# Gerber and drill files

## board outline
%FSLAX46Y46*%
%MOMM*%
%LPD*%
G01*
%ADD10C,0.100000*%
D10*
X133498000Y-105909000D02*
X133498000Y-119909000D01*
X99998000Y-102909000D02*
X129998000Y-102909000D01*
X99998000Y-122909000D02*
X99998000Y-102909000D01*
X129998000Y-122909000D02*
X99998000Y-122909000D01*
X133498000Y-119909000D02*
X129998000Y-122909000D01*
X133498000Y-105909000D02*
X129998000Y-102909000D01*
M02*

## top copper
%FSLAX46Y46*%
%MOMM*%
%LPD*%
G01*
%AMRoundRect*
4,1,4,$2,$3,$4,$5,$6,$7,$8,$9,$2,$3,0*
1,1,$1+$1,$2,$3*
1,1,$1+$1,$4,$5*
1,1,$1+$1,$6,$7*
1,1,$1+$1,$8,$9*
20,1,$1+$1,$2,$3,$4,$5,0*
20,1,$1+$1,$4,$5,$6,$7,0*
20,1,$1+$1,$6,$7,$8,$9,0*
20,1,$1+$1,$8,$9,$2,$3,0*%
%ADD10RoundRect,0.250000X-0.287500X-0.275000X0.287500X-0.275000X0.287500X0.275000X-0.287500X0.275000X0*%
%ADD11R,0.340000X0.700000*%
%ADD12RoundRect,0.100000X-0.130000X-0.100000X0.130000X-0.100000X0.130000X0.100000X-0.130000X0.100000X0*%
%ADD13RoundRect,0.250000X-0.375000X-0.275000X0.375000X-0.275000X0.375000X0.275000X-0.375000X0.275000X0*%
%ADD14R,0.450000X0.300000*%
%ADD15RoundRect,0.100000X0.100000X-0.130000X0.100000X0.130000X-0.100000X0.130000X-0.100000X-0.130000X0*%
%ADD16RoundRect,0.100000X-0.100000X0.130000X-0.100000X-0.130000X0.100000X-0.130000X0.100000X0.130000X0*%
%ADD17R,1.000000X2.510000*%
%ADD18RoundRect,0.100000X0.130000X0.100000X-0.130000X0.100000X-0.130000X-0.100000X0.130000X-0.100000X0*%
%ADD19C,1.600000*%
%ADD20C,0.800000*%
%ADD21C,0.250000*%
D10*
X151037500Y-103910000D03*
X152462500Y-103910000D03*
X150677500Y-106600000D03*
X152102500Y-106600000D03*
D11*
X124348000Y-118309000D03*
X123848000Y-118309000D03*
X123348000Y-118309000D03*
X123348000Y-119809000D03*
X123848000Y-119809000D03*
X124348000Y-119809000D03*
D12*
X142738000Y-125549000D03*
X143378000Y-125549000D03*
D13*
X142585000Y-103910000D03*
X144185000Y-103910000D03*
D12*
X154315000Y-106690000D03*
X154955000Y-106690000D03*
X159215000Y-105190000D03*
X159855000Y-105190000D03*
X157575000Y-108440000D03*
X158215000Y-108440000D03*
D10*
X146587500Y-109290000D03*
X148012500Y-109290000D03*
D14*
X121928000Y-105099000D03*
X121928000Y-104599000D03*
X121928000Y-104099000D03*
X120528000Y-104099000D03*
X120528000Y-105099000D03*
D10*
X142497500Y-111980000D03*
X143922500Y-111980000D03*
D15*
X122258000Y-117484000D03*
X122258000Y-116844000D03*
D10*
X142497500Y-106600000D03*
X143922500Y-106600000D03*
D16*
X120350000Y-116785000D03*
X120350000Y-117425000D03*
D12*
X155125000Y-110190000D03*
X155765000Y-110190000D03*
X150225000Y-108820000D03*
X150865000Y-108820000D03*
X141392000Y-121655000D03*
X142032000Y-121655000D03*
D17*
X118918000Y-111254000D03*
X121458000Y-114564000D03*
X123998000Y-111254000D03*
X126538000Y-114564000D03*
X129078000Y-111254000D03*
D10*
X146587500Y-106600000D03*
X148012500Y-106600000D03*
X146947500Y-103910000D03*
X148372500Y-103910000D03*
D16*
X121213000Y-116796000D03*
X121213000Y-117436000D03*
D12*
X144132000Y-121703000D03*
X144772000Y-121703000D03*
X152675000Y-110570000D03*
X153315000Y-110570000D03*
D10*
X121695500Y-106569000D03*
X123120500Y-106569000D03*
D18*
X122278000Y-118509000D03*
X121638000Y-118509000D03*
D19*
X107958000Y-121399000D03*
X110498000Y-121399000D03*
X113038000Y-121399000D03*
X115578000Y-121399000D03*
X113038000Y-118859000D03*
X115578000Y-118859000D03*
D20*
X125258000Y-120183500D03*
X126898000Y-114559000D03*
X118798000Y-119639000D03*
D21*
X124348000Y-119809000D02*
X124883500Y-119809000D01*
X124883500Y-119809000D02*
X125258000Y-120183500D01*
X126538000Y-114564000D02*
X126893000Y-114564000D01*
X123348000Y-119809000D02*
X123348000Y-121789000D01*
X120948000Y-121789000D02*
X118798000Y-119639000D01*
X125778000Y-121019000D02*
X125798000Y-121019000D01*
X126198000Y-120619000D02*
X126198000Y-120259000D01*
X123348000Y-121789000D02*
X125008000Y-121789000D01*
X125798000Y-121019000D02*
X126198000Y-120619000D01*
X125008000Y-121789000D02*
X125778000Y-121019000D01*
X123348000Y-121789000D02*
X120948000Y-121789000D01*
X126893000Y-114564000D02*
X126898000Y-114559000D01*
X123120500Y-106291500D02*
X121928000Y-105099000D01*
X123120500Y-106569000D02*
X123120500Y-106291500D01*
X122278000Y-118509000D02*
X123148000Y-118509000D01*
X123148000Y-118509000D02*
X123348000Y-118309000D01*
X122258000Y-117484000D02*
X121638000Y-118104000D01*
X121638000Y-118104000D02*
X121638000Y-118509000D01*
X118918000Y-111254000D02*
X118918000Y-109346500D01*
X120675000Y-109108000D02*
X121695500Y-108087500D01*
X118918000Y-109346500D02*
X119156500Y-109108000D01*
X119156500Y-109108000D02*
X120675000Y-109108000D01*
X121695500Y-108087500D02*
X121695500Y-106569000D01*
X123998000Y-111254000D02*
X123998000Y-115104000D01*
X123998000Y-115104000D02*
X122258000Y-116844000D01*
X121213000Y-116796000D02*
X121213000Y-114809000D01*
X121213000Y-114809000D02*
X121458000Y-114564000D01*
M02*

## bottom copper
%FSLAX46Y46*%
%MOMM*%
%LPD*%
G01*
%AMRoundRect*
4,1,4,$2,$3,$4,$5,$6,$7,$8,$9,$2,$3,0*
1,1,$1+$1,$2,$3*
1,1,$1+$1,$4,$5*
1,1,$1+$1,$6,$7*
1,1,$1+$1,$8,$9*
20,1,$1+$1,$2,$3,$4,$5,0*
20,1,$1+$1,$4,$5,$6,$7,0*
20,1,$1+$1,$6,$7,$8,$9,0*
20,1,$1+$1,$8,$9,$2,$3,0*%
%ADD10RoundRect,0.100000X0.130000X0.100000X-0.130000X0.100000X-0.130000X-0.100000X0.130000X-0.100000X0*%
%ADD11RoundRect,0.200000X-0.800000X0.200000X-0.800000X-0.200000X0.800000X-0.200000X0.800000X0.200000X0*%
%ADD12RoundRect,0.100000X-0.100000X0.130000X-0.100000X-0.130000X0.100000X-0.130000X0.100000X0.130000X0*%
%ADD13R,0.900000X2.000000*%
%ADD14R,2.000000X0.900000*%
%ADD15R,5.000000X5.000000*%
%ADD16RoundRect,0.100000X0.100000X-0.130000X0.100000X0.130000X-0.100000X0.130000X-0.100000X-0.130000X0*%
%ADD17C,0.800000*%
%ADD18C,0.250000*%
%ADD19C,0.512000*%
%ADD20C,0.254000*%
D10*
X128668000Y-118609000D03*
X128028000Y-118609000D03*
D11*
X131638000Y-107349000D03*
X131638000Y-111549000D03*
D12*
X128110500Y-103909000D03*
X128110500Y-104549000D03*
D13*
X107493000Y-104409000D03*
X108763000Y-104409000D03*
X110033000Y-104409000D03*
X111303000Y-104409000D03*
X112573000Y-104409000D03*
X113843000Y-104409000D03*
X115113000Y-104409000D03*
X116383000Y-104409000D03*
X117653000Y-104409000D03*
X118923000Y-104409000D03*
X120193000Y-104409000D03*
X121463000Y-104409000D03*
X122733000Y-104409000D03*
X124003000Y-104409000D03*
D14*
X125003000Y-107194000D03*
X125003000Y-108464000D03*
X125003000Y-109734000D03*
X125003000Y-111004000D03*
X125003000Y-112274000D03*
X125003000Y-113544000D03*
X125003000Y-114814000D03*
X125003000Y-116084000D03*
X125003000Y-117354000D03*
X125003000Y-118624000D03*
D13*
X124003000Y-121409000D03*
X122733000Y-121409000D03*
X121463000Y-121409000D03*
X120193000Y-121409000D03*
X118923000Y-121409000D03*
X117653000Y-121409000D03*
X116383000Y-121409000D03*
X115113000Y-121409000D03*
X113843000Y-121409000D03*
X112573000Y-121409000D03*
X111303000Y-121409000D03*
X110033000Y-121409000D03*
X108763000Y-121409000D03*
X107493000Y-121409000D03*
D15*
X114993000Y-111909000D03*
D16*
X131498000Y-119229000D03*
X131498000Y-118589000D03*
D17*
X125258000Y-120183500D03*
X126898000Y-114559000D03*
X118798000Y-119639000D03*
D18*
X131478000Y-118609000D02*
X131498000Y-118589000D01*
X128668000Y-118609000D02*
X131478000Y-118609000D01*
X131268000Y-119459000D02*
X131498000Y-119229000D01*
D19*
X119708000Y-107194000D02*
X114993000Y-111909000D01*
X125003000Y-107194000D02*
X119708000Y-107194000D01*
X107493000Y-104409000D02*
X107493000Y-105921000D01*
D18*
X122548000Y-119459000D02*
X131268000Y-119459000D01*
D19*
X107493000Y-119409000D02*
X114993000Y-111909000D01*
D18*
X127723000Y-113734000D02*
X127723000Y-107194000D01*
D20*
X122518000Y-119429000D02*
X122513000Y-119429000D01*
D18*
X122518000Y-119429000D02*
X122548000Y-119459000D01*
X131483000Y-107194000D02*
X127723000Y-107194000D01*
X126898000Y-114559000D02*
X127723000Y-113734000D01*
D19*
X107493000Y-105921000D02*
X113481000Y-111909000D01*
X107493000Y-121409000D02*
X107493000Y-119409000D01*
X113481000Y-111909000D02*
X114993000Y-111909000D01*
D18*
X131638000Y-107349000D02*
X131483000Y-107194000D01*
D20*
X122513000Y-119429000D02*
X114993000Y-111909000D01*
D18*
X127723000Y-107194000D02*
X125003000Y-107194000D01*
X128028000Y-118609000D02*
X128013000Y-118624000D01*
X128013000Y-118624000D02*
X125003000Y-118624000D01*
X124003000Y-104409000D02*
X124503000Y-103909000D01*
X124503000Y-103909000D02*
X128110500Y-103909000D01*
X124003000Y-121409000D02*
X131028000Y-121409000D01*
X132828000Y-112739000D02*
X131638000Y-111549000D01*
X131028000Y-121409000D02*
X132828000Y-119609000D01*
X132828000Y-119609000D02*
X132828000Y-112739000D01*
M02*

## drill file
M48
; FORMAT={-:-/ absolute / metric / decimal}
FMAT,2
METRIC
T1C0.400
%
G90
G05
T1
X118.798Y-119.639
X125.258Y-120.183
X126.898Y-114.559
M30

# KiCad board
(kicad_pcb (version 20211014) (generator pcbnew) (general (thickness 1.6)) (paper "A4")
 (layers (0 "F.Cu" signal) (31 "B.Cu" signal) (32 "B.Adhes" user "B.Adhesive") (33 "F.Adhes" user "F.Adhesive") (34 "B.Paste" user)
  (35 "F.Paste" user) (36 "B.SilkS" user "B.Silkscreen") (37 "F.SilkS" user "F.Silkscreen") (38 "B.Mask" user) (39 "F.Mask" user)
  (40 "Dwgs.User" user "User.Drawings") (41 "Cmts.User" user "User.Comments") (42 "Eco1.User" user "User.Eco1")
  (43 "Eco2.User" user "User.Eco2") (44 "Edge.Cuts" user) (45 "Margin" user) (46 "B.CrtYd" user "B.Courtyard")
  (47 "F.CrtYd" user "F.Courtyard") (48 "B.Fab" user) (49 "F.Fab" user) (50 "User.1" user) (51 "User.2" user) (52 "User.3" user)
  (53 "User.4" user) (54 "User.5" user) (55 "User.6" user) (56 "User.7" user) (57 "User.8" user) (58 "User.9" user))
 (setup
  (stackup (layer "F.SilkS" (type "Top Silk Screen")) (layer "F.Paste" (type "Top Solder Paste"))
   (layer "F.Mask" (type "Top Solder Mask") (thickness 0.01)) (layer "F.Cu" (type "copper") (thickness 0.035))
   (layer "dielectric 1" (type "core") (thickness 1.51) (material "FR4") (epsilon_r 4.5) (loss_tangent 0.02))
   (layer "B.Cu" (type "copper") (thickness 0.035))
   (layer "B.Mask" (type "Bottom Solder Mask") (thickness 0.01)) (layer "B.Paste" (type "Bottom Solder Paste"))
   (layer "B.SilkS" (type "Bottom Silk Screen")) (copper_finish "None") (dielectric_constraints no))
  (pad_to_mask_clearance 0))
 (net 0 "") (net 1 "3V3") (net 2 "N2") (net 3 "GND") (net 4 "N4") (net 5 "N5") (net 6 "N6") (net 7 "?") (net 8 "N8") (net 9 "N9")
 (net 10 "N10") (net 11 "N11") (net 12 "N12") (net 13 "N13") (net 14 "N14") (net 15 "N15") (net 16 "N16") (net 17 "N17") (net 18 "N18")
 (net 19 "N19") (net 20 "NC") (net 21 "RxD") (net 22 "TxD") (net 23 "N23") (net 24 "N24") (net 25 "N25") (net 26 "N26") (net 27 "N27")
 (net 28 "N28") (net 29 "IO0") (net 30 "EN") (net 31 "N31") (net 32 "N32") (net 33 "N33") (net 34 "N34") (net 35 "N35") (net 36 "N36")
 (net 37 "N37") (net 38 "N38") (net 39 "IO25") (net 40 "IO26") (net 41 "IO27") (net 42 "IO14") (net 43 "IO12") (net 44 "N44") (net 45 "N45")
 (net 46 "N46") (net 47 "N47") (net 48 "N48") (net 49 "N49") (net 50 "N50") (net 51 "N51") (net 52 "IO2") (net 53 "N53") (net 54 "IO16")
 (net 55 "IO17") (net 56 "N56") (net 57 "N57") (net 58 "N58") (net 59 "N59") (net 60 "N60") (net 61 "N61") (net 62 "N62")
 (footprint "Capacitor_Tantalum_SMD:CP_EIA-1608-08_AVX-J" (layer "F.Cu") (at 151.75 103.91)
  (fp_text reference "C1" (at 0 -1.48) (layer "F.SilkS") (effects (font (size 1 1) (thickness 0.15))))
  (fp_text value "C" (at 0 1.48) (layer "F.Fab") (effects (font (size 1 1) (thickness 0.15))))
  (pad "1" smd roundrect (at -0.7125 0) (size 1.075 1.05) (layers "F.Cu" "F.Paste" "F.Mask") (roundrect_rratio 0.238095) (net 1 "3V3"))
  (pad "2" smd roundrect (at 0.7125 0) (size 1.075 1.05) (layers "F.Cu" "F.Paste" "F.Mask") (roundrect_rratio 0.238095) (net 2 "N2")))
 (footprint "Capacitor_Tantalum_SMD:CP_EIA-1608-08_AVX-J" (layer "F.Cu") (at 151.39 106.6)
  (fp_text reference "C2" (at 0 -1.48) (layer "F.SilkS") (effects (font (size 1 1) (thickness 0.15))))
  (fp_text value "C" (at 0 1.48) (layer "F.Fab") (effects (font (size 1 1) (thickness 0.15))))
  (pad "1" smd roundrect (at -0.7125 0) (size 1.075 1.05) (layers "F.Cu" "F.Paste" "F.Mask") (roundrect_rratio 0.238095) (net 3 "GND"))
  (pad "2" smd roundrect (at 0.7125 0) (size 1.075 1.05) (layers "F.Cu" "F.Paste" "F.Mask") (roundrect_rratio 0.238095) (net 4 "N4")))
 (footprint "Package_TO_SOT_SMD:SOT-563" (layer "F.Cu") (at 123.848 119.059 -90)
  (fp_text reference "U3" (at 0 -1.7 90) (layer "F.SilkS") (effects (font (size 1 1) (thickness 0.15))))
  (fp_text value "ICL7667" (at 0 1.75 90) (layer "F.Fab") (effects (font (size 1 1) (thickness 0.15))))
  (pad "1" smd rect (at -0.75 -0.5 270) (size 0.7 0.34) (layers "F.Cu" "F.Paste" "F.Mask") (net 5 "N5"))
  (pad "2" smd rect (at -0.75 0 270) (size 0.7 0.34) (layers "F.Cu" "F.Paste" "F.Mask") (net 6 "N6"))
  (pad "3" smd rect (at -0.75 0.5 270) (size 0.7 0.34) (layers "F.Cu" "F.Paste" "F.Mask") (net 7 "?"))
  (pad "4" smd rect (at 0.75 0.5 270) (size 0.7 0.34) (layers "F.Cu" "F.Paste" "F.Mask") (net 3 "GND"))
  (pad "5" smd rect (at 0.75 0 270) (size 0.7 0.34) (layers "F.Cu" "F.Paste" "F.Mask") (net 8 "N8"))
  (pad "6" smd rect (at 0.75 -0.5 270) (size 0.7 0.34) (layers "F.Cu" "F.Paste" "F.Mask") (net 1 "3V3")))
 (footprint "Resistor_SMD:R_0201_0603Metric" (layer "F.Cu") (at 143.058 125.549)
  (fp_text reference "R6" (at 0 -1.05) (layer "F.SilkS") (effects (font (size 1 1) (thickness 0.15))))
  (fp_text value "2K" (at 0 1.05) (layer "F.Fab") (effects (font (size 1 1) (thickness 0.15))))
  (pad "" smd roundrect (at -0.345 0) (size 0.318 0.36) (layers "F.Paste") (roundrect_rratio 0.25))
  (pad "" smd roundrect (at 0.345 0) (size 0.318 0.36) (layers "F.Paste") (roundrect_rratio 0.25))
  (pad "1" smd roundrect (at -0.32 0) (size 0.46 0.4) (layers "F.Cu" "F.Mask") (roundrect_rratio 0.25) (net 3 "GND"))
  (pad "2" smd roundrect (at 0.32 0) (size 0.46 0.4) (layers "F.Cu" "F.Mask") (roundrect_rratio 0.25) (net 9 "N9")))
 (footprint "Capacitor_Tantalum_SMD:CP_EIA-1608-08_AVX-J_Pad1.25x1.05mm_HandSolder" (layer "F.Cu") (at 143.385 103.91)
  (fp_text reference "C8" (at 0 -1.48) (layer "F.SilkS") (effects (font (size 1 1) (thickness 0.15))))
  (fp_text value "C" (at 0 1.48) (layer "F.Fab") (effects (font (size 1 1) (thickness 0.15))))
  (pad "1" smd roundrect (at -0.8 0) (size 1.25 1.05) (layers "F.Cu" "F.Paste" "F.Mask") (roundrect_rratio 0.238095) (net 1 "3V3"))
  (pad "2" smd roundrect (at 0.8 0) (size 1.25 1.05) (layers "F.Cu" "F.Paste" "F.Mask") (roundrect_rratio 0.238095) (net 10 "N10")))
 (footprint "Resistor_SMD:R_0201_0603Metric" (layer "F.Cu") (at 154.635 106.69)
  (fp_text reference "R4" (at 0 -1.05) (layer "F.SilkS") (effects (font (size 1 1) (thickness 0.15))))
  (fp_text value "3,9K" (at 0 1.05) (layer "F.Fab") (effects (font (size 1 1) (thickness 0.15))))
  (pad "" smd roundrect (at 0.345 0) (size 0.318 0.36) (layers "F.Paste") (roundrect_rratio 0.25))
  (pad "" smd roundrect (at -0.345 0) (size 0.318 0.36) (layers "F.Paste") (roundrect_rratio 0.25))
  (pad "1" smd roundrect (at -0.32 0) (size 0.46 0.4) (layers "F.Cu" "F.Mask") (roundrect_rratio 0.25) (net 3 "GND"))
  (pad "2" smd roundrect (at 0.32 0) (size 0.46 0.4) (layers "F.Cu" "F.Mask") (roundrect_rratio 0.25) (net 2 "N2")))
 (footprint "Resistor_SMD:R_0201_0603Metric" (layer "F.Cu") (at 159.535 105.19)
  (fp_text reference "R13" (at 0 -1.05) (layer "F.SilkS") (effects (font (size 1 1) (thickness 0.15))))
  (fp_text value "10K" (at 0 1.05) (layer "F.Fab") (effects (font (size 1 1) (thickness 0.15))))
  (pad "" smd roundrect (at 0.345 0) (size 0.318 0.36) (layers "F.Paste") (roundrect_rratio 0.25))
  (pad "" smd roundrect (at -0.345 0) (size 0.318 0.36) (layers "F.Paste") (roundrect_rratio 0.25))
  (pad "1" smd roundrect (at -0.32 0) (size 0.46 0.4) (layers "F.Cu" "F.Mask") (roundrect_rratio 0.25) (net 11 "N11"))
  (pad "2" smd roundrect (at 0.32 0) (size 0.46 0.4) (layers "F.Cu" "F.Mask") (roundrect_rratio 0.25) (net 1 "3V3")))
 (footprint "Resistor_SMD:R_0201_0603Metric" (layer "F.Cu") (at 157.895 108.44)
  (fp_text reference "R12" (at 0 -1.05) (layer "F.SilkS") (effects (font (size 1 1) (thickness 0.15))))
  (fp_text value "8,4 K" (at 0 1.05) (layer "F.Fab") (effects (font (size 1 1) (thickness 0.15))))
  (pad "" smd roundrect (at -0.345 0) (size 0.318 0.36) (layers "F.Paste") (roundrect_rratio 0.25))
  (pad "" smd roundrect (at 0.345 0) (size 0.318 0.36) (layers "F.Paste") (roundrect_rratio 0.25))
  (pad "1" smd roundrect (at -0.32 0) (size 0.46 0.4) (layers "F.Cu" "F.Mask") (roundrect_rratio 0.25) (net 1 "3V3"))
  (pad "2" smd roundrect (at 0.32 0) (size 0.46 0.4) (layers "F.Cu" "F.Mask") (roundrect_rratio 0.25) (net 8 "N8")))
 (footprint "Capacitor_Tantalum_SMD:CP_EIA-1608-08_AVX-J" (layer "F.Cu") (at 147.3 109.29)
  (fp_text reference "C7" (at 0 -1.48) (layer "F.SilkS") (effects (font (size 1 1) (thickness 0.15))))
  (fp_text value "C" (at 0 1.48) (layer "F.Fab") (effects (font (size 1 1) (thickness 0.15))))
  (pad "1" smd roundrect (at -0.7125 0) (size 1.075 1.05) (layers "F.Cu" "F.Paste" "F.Mask") (roundrect_rratio 0.238095) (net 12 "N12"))
  (pad "2" smd roundrect (at 0.7125 0) (size 1.075 1.05) (layers "F.Cu" "F.Paste" "F.Mask") (roundrect_rratio 0.238095) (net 1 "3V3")))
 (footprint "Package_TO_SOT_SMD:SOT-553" (layer "F.Cu") (at 121.228 104.599 180)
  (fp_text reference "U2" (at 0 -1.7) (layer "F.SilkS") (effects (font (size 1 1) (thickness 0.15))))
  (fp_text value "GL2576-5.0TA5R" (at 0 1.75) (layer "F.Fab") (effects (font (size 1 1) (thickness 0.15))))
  (pad "1" smd rect (at -0.7 -0.5 180) (size 0.45 0.3) (layers "F.Cu" "F.Paste" "F.Mask") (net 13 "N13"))
  (pad "2" smd rect (at -0.7 0 180) (size 0.45 0.3) (layers "F.Cu" "F.Paste" "F.Mask") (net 3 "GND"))
  (pad "3" smd rect (at -0.7 0.5 180) (size 0.45 0.3) (layers "F.Cu" "F.Paste" "F.Mask") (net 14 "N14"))
  (pad "4" smd rect (at 0.7 0.5 180) (size 0.45 0.3) (layers "F.Cu" "F.Paste" "F.Mask") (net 4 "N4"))
  (pad "5" smd rect (at 0.7 -0.5 180) (size 0.45 0.3) (layers "F.Cu" "F.Paste" "F.Mask") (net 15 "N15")))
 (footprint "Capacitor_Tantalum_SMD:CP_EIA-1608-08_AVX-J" (layer "F.Cu") (at 143.21 111.98)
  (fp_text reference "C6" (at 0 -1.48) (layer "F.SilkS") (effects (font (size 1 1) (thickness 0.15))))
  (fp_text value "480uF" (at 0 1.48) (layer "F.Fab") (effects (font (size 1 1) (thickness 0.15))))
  (pad "1" smd roundrect (at -0.7125 0) (size 1.075 1.05) (layers "F.Cu" "F.Paste" "F.Mask") (roundrect_rratio 0.238095) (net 3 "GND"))
  (pad "2" smd roundrect (at 0.7125 0) (size 1.075 1.05) (layers "F.Cu" "F.Paste" "F.Mask") (roundrect_rratio 0.238095) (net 1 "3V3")))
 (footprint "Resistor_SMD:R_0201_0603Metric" (layer "F.Cu") (at 122.258 117.164 90)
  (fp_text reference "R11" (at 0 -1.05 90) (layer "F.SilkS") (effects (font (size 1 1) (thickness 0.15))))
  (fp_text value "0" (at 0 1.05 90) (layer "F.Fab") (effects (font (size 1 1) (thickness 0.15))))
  (pad "" smd roundrect (at -0.345 0 90) (size 0.318 0.36) (layers "F.Paste") (roundrect_rratio 0.25))
  (pad "" smd roundrect (at 0.345 0 90) (size 0.318 0.36) (layers "F.Paste") (roundrect_rratio 0.25))
  (pad "1" smd roundrect (at -0.32 0 90) (size 0.46 0.4) (layers "F.Cu" "F.Mask") (roundrect_rratio 0.25) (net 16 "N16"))
  (pad "2" smd roundrect (at 0.32 0 90) (size 0.46 0.4) (layers "F.Cu" "F.Mask") (roundrect_rratio 0.25) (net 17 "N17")))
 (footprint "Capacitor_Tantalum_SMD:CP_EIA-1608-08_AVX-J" (layer "F.Cu") (at 143.21 106.6)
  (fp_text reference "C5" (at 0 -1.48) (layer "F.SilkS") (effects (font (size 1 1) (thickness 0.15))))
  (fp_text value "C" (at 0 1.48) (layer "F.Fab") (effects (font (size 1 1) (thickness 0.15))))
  (pad "1" smd roundrect (at -0.7125 0) (size 1.075 1.05) (layers "F.Cu" "F.Paste" "F.Mask") (roundrect_rratio 0.238095) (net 3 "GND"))
  (pad "2" smd roundrect (at 0.7125 0) (size 1.075 1.05) (layers "F.Cu" "F.Paste" "F.Mask") (roundrect_rratio 0.238095) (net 6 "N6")))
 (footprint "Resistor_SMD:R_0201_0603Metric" (layer "F.Cu") (at 120.35 117.105 -90)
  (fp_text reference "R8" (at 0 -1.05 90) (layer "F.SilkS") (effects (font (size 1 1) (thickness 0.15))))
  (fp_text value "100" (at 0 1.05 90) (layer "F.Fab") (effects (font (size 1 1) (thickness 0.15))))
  (pad "" smd roundrect (at 0.345 0 270) (size 0.318 0.36) (layers "F.Paste") (roundrect_rratio 0.25))
  (pad "" smd roundrect (at -0.345 0 270) (size 0.318 0.36) (layers "F.Paste") (roundrect_rratio 0.25))
  (pad "1" smd roundrect (at -0.32 0 270) (size 0.46 0.4) (layers "F.Cu" "F.Mask") (roundrect_rratio 0.25) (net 1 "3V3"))
  (pad "2" smd roundrect (at 0.32 0 270) (size 0.46 0.4) (layers "F.Cu" "F.Mask") (roundrect_rratio 0.25) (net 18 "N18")))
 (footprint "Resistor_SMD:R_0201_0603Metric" (layer "F.Cu") (at 155.445 110.19)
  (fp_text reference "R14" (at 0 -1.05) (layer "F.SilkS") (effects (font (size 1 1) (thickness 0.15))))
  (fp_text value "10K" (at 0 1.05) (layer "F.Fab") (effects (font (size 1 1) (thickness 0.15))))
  (pad "" smd roundrect (at -0.345 0) (size 0.318 0.36) (layers "F.Paste") (roundrect_rratio 0.25))
  (pad "" smd roundrect (at 0.345 0) (size 0.318 0.36) (layers "F.Paste") (roundrect_rratio 0.25))
  (pad "1" smd roundrect (at -0.32 0) (size 0.46 0.4) (layers "F.Cu" "F.Mask") (roundrect_rratio 0.25) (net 3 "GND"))
  (pad "2" smd roundrect (at 0.32 0) (size 0.46 0.4) (layers "F.Cu" "F.Mask") (roundrect_rratio 0.25) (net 1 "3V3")))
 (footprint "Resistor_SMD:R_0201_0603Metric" (layer "F.Cu") (at 150.545 108.82)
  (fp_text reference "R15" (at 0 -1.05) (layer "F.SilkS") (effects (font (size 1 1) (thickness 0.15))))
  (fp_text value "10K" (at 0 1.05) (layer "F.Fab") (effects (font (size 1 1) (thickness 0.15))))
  (pad "" smd roundrect (at -0.345 0) (size 0.318 0.36) (layers "F.Paste") (roundrect_rratio 0.25))
  (pad "" smd roundrect (at 0.345 0) (size 0.318 0.36) (layers "F.Paste") (roundrect_rratio 0.25))
  (pad "1" smd roundrect (at -0.32 0) (size 0.46 0.4) (layers "F.Cu" "F.Mask") (roundrect_rratio 0.25) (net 1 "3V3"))
  (pad "2" smd roundrect (at 0.32 0) (size 0.46 0.4) (layers "F.Cu" "F.Mask") (roundrect_rratio 0.25) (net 12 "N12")))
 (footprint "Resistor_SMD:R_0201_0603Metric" (layer "F.Cu") (at 141.712 121.655)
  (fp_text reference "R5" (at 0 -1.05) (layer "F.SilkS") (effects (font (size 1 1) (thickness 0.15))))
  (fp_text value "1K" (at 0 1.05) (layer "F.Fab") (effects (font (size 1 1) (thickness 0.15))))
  (pad "" smd roundrect (at 0.345 0) (size 0.318 0.36) (layers "F.Paste") (roundrect_rratio 0.25))
  (pad "" smd roundrect (at -0.345 0) (size 0.318 0.36) (layers "F.Paste") (roundrect_rratio 0.25))
  (pad "1" smd roundrect (at -0.32 0) (size 0.46 0.4) (layers "F.Cu" "F.Mask") (roundrect_rratio 0.25) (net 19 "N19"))
  (pad "2" smd roundrect (at 0.32 0) (size 0.46 0.4) (layers "F.Cu" "F.Mask") (roundrect_rratio 0.25) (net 9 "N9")))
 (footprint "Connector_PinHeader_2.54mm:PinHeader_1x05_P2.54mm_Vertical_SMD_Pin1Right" (layer "F.Cu") (at 123.998 112.909 90)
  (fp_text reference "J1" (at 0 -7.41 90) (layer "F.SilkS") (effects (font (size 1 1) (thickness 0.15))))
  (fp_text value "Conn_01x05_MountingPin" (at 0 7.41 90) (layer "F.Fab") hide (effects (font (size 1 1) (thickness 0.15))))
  (pad "+5V" smd rect (at 1.655 -5.08 90) (size 2.51 1) (layers "F.Cu" "F.Paste" "F.Mask"))
  (pad "2" smd rect (at -1.655 -2.54 90) (size 2.51 1) (layers "F.Cu" "F.Paste" "F.Mask") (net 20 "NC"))
  (pad "3" smd rect (at 1.655 0 90) (size 2.51 1) (layers "F.Cu" "F.Paste" "F.Mask") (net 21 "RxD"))
  (pad "4" smd rect (at -1.655 2.54 90) (size 2.51 1) (layers "F.Cu" "F.Paste" "F.Mask") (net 3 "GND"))
  (pad "5" smd rect (at 1.655 5.08 90) (size 2.51 1) (layers "F.Cu" "F.Paste" "F.Mask") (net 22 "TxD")))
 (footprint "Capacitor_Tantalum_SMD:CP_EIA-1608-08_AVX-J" (layer "F.Cu") (at 147.3 106.6)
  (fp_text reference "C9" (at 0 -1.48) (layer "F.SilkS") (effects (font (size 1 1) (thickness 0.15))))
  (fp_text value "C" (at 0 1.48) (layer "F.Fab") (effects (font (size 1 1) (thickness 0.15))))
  (pad "1" smd roundrect (at -0.7125 0) (size 1.075 1.05) (layers "F.Cu" "F.Paste" "F.Mask") (roundrect_rratio 0.238095) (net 10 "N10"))
  (pad "2" smd roundrect (at 0.7125 0) (size 1.075 1.05) (layers "F.Cu" "F.Paste" "F.Mask") (roundrect_rratio 0.238095) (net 3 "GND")))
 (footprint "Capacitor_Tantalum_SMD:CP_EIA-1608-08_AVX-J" (layer "F.Cu") (at 147.66 103.91)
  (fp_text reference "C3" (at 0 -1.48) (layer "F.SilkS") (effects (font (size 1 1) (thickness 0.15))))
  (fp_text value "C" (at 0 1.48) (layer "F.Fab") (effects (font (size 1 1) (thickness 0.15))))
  (pad "1" smd roundrect (at -0.7125 0) (size 1.075 1.05) (layers "F.Cu" "F.Paste" "F.Mask") (roundrect_rratio 0.238095) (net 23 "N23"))
  (pad "2" smd roundrect (at 0.7125 0) (size 1.075 1.05) (layers "F.Cu" "F.Paste" "F.Mask") (roundrect_rratio 0.238095) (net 1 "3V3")))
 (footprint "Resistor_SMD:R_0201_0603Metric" (layer "F.Cu") (at 121.213 117.116 -90)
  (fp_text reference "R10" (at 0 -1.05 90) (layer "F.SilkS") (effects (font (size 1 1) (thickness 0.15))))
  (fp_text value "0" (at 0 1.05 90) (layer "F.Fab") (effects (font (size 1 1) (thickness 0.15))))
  (pad "" smd roundrect (at 0.345 0 270) (size 0.318 0.36) (layers "F.Paste") (roundrect_rratio 0.25))
  (pad "" smd roundrect (at -0.345 0 270) (size 0.318 0.36) (layers "F.Paste") (roundrect_rratio 0.25))
  (pad "1" smd roundrect (at -0.32 0 270) (size 0.46 0.4) (layers "F.Cu" "F.Mask") (roundrect_rratio 0.25) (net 20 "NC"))
  (pad "2" smd roundrect (at 0.32 0 270) (size 0.46 0.4) (layers "F.Cu" "F.Mask") (roundrect_rratio 0.25) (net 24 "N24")))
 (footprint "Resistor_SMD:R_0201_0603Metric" (layer "F.Cu") (at 144.452 121.703)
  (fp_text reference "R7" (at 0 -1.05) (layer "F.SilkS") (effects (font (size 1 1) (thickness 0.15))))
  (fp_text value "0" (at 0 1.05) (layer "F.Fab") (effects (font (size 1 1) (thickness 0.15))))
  (pad "" smd roundrect (at 0.345 0) (size 0.318 0.36) (layers "F.Paste") (roundrect_rratio 0.25))
  (pad "" smd roundrect (at -0.345 0) (size 0.318 0.36) (layers "F.Paste") (roundrect_rratio 0.25))
  (pad "1" smd roundrect (at -0.32 0) (size 0.46 0.4) (layers "F.Cu" "F.Mask") (roundrect_rratio 0.25) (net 9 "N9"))
  (pad "2" smd roundrect (at 0.32 0) (size 0.46 0.4) (layers "F.Cu" "F.Mask") (roundrect_rratio 0.25) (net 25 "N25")))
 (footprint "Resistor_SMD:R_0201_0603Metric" (layer "F.Cu") (at 152.995 110.57)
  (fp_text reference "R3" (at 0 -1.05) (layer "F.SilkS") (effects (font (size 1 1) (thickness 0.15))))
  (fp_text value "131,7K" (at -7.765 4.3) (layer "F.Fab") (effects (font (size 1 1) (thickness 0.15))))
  (pad "" smd roundrect (at 0.345 0) (size 0.318 0.36) (layers "F.Paste") (roundrect_rratio 0.25))
  (pad "" smd roundrect (at -0.345 0) (size 0.318 0.36) (layers "F.Paste") (roundrect_rratio 0.25))
  (pad "1" smd roundrect (at -0.32 0) (size 0.46 0.4) (layers "F.Cu" "F.Mask") (roundrect_rratio 0.25) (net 2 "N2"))
  (pad "2" smd roundrect (at 0.32 0) (size 0.46 0.4) (layers "F.Cu" "F.Mask") (roundrect_rratio 0.25) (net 1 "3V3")))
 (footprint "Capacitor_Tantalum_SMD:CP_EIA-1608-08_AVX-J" (layer "F.Cu") (at 122.408 106.569)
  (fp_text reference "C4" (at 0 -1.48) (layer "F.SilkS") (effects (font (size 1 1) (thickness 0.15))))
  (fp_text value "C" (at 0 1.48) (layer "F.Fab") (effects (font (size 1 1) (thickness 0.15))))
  (pad "1" smd roundrect (at -0.7125 0) (size 1.075 1.05) (layers "F.Cu" "F.Paste" "F.Mask") (roundrect_rratio 0.238095) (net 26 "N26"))
  (pad "2" smd roundrect (at 0.7125 0) (size 1.075 1.05) (layers "F.Cu" "F.Paste" "F.Mask") (roundrect_rratio 0.238095) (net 13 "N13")))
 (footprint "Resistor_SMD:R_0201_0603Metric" (layer "F.Cu") (at 121.958 118.509 180)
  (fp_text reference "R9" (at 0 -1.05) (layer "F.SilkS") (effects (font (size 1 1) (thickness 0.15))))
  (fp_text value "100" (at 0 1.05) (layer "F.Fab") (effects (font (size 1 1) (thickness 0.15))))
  (pad "" smd roundrect (at 0.345 0 180) (size 0.318 0.36) (layers "F.Paste") (roundrect_rratio 0.25))
  (pad "" smd roundrect (at -0.345 0 180) (size 0.318 0.36) (layers "F.Paste") (roundrect_rratio 0.25))
  (pad "1" smd roundrect (at -0.32 0 180) (size 0.46 0.4) (layers "F.Cu" "F.Mask") (roundrect_rratio 0.25) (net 7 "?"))
  (pad "2" smd roundrect (at 0.32 0 180) (size 0.46 0.4) (layers "F.Cu" "F.Mask") (roundrect_rratio 0.25) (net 16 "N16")))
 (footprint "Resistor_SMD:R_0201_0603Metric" (layer "B.Cu") (at 128.348 118.609 180)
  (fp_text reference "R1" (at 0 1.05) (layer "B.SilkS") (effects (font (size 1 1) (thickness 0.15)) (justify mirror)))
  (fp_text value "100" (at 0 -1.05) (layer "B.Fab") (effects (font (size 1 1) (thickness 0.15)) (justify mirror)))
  (pad "" smd roundrect (at -0.345 0 180) (size 0.318 0.36) (layers "B.Paste") (roundrect_rratio 0.25))
  (pad "" smd roundrect (at 0.345 0 180) (size 0.318 0.36) (layers "B.Paste") (roundrect_rratio 0.25))
  (pad "1" smd roundrect (at -0.32 0 180) (size 0.46 0.4) (layers "B.Cu" "B.Mask") (roundrect_rratio 0.25) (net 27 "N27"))
  (pad "2" smd roundrect (at 0.32 0 180) (size 0.46 0.4) (layers "B.Cu" "B.Mask") (roundrect_rratio 0.25) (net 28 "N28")))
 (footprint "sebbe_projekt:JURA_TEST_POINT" (layer "B.Cu") (at 107.958 121.399)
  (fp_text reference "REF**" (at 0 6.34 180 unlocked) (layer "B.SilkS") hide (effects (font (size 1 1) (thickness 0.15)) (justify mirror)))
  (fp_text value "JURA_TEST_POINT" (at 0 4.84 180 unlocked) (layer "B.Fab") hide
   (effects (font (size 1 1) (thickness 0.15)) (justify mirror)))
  (pad "1" smd circle (at 0 0) (size 1.6 1.6) (layers "F.Cu" "B.Paste" "B.Mask") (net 3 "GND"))
  (pad "2" smd circle (at 2.54 0) (size 1.6 1.6) (layers "F.Cu" "B.Paste" "B.Mask") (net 22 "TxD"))
  (pad "3" smd circle (at 5.08 0) (size 1.6 1.6) (layers "F.Cu" "B.Paste" "B.Mask") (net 21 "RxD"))
  (pad "4" smd circle (at 7.62 0) (size 1.6 1.6) (layers "F.Cu" "B.Paste" "B.Mask") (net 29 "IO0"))
  (pad "5" smd circle (at 5.08 -2.54) (size 1.6 1.6) (layers "F.Cu" "B.Paste" "B.Mask") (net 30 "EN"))
  (pad "6" smd circle (at 7.62 -2.54) (size 1.6 1.6) (layers "F.Cu" "B.Paste" "B.Mask") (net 1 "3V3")))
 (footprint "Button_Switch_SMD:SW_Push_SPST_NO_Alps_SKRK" (layer "B.Cu") (at 131.638 109.449 -90)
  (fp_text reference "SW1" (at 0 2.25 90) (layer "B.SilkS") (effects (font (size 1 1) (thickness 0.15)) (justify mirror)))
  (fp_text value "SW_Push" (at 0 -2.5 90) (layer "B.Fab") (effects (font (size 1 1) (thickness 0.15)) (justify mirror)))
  (pad "1" smd roundrect (at -2.1 0 270) (size 0.8 2) (layers "B.Cu" "B.Paste" "B.Mask") (roundrect_rratio 0.25) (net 3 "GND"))
  (pad "2" smd roundrect (at 2.1 0 270) (size 0.8 2) (layers "B.Cu" "B.Paste" "B.Mask") (roundrect_rratio 0.25) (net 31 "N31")))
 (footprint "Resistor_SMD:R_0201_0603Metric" (layer "B.Cu") (at 128.1105 104.229 -90)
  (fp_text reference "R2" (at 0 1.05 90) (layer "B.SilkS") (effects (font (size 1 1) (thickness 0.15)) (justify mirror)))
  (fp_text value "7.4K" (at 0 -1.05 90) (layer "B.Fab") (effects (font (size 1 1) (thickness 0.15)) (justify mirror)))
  (pad "" smd roundrect (at 0.345 0 270) (size 0.318 0.36) (layers "B.Paste") (roundrect_rratio 0.25))
  (pad "" smd roundrect (at -0.345 0 270) (size 0.318 0.36) (layers "B.Paste") (roundrect_rratio 0.25))
  (pad "1" smd roundrect (at -0.32 0 270) (size 0.46 0.4) (layers "B.Cu" "B.Mask") (roundrect_rratio 0.25) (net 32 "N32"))
  (pad "2" smd roundrect (at 0.32 0 270) (size 0.46 0.4) (layers "B.Cu" "B.Mask") (roundrect_rratio 0.25) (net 3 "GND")))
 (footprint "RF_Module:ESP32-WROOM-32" (layer "B.Cu") (at 115.748 112.909 -90)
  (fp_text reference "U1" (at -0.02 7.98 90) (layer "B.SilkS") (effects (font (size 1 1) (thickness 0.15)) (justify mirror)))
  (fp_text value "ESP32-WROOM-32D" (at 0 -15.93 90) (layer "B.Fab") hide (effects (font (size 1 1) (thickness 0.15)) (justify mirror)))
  (pad "1" smd rect (at -8.5 8.255 270) (size 2 0.9) (layers "B.Cu" "B.Paste" "B.Mask") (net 3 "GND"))
  (pad "2" smd rect (at -8.5 6.985 270) (size 2 0.9) (layers "B.Cu" "B.Paste" "B.Mask") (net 1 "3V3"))
  (pad "3" smd rect (at -8.5 5.715 270) (size 2 0.9) (layers "B.Cu" "B.Paste" "B.Mask") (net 30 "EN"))
  (pad "4" smd rect (at -8.5 4.445 270) (size 2 0.9) (layers "B.Cu" "B.Paste" "B.Mask") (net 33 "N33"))
  (pad "5" smd rect (at -8.5 3.175 270) (size 2 0.9) (layers "B.Cu" "B.Paste" "B.Mask") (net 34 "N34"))
  (pad "6" smd rect (at -8.5 1.905 270) (size 2 0.9) (layers "B.Cu" "B.Paste" "B.Mask") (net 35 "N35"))
  (pad "7" smd rect (at -8.5 0.635 270) (size 2 0.9) (layers "B.Cu" "B.Paste" "B.Mask") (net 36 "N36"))
  (pad "8" smd rect (at -8.5 -0.635 270) (size 2 0.9) (layers "B.Cu" "B.Paste" "B.Mask") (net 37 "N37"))
  (pad "9" smd rect (at -8.5 -1.905 270) (size 2 0.9) (layers "B.Cu" "B.Paste" "B.Mask") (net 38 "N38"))
  (pad "10" smd rect (at -8.5 -3.175 270) (size 2 0.9) (layers "B.Cu" "B.Paste" "B.Mask") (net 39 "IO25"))
  (pad "11" smd rect (at -8.5 -4.445 270) (size 2 0.9) (layers "B.Cu" "B.Paste" "B.Mask") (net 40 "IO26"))
  (pad "12" smd rect (at -8.5 -5.715 270) (size 2 0.9) (layers "B.Cu" "B.Paste" "B.Mask") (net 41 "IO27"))
  (pad "13" smd rect (at -8.5 -6.985 270) (size 2 0.9) (layers "B.Cu" "B.Paste" "B.Mask") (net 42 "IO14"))
  (pad "14" smd rect (at -8.5 -8.255 270) (size 2 0.9) (layers "B.Cu" "B.Paste" "B.Mask") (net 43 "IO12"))
  (pad "15" smd rect (at -5.715 -9.255 180) (size 2 0.9) (layers "B.Cu" "B.Paste" "B.Mask") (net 3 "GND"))
  (pad "16" smd rect (at -4.445 -9.255 180) (size 2 0.9) (layers "B.Cu" "B.Paste" "B.Mask") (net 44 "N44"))
  (pad "17" smd rect (at -3.175 -9.255 180) (size 2 0.9) (layers "B.Cu" "B.Paste" "B.Mask") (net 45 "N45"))
  (pad "18" smd rect (at -1.905 -9.255 180) (size 2 0.9) (layers "B.Cu" "B.Paste" "B.Mask") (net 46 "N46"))
  (pad "19" smd rect (at -0.635 -9.255 180) (size 2 0.9) (layers "B.Cu" "B.Paste" "B.Mask") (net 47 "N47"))
  (pad "20" smd rect (at 0.635 -9.255 180) (size 2 0.9) (layers "B.Cu" "B.Paste" "B.Mask") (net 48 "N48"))
  (pad "21" smd rect (at 1.905 -9.255 180) (size 2 0.9) (layers "B.Cu" "B.Paste" "B.Mask") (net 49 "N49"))
  (pad "22" smd rect (at 3.175 -9.255 180) (size 2 0.9) (layers "B.Cu" "B.Paste" "B.Mask") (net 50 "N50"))
  (pad "23" smd rect (at 4.445 -9.255 180) (size 2 0.9) (layers "B.Cu" "B.Paste" "B.Mask") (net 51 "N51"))
  (pad "24" smd rect (at 5.715 -9.255 180) (size 2 0.9) (layers "B.Cu" "B.Paste" "B.Mask") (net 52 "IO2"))
  (pad "25" smd rect (at 8.5 -8.255 270) (size 2 0.9) (layers "B.Cu" "B.Paste" "B.Mask") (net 29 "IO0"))
  (pad "26" smd rect (at 8.5 -6.985 270) (size 2 0.9) (layers "B.Cu" "B.Paste" "B.Mask") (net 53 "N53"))
  (pad "27" smd rect (at 8.5 -5.715 270) (size 2 0.9) (layers "B.Cu" "B.Paste" "B.Mask") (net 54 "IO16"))
  (pad "28" smd rect (at 8.5 -4.445 270) (size 2 0.9) (layers "B.Cu" "B.Paste" "B.Mask") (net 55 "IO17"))
  (pad "29" smd rect (at 8.5 -3.175 270) (size 2 0.9) (layers "B.Cu" "B.Paste" "B.Mask") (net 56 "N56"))
  (pad "30" smd rect (at 8.5 -1.905 270) (size 2 0.9) (layers "B.Cu" "B.Paste" "B.Mask") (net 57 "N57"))
  (pad "31" smd rect (at 8.5 -0.635 270) (size 2 0.9) (layers "B.Cu" "B.Paste" "B.Mask") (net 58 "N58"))
  (pad "32" smd rect (at 8.5 0.635 270) (size 2 0.9) (layers "B.Cu" "B.Paste" "B.Mask") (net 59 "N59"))
  (pad "33" smd rect (at 8.5 1.905 270) (size 2 0.9) (layers "B.Cu" "B.Paste" "B.Mask") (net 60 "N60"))
  (pad "34" smd rect (at 8.5 3.175 270) (size 2 0.9) (layers "B.Cu" "B.Paste" "B.Mask") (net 21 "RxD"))
  (pad "35" smd rect (at 8.5 4.445 270) (size 2 0.9) (layers "B.Cu" "B.Paste" "B.Mask") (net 22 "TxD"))
  (pad "36" smd rect (at 8.5 5.715 270) (size 2 0.9) (layers "B.Cu" "B.Paste" "B.Mask") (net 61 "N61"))
  (pad "37" smd rect (at 8.5 6.985 270) (size 2 0.9) (layers "B.Cu" "B.Paste" "B.Mask") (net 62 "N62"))
  (pad "38" smd rect (at 8.5 8.255 270) (size 2 0.9) (layers "B.Cu" "B.Paste" "B.Mask") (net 3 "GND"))
  (pad "39" smd rect (at -1 0.755 270) (size 5 5) (layers "B.Cu" "B.Paste" "B.Mask") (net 3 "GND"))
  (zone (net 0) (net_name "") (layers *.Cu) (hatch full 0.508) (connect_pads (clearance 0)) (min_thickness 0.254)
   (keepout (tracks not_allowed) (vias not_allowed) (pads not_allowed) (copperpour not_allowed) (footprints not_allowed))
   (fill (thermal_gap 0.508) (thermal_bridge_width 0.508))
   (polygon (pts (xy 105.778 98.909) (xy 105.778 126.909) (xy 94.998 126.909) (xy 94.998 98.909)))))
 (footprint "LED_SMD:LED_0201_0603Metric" (layer "B.Cu") (at 131.498 118.909 90)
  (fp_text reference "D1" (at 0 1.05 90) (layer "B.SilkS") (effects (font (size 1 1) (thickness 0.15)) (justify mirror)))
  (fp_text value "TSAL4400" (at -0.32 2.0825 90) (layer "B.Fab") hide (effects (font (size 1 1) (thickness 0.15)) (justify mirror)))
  (pad "" smd roundrect (at 0.345 0 90) (size 0.318 0.36) (layers "B.Paste") (roundrect_rratio 0.25))
  (pad "" smd roundrect (at -0.345 0 90) (size 0.318 0.36) (layers "B.Paste") (roundrect_rratio 0.25))
  (pad "1" smd roundrect (at -0.32 0 90) (size 0.46 0.4) (layers "B.Cu" "B.Mask") (roundrect_rratio 0.25) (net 3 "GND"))
  (pad "2" smd roundrect (at 0.32 0 90) (size 0.46 0.4) (layers "B.Cu" "B.Mask") (roundrect_rratio 0.25) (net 27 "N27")))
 (gr_line (start 133.498 105.909) (end 133.498 119.909) (layer "Edge.Cuts") (width 0.1))
 (gr_line (start 99.998 102.909) (end 129.998 102.909) (layer "Edge.Cuts") (width 0.1))
 (gr_line (start 99.998 122.909) (end 99.998 102.909) (layer "Edge.Cuts") (width 0.1))
 (gr_line (start 129.998 122.909) (end 99.998 122.909) (layer "Edge.Cuts") (width 0.1))
 (gr_line (start 133.498 119.909) (end 129.998 122.909) (layer "Edge.Cuts") (width 0.1))
 (gr_line (start 133.498 105.909) (end 129.998 102.909) (layer "Edge.Cuts") (width 0.1))
 (segment (start 124.348 119.809) (end 124.8835 119.809) (width 0.25) (layer "F.Cu") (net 1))
 (segment (start 124.8835 119.809) (end 125.258 120.1835) (width 0.25) (layer "F.Cu") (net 1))
 (via (at 125.258 120.1835) (size 0.8) (drill 0.4) (layers "F.Cu" "B.Cu") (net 1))
 (segment (start 131.478 118.609) (end 131.498 118.589) (width 0.25) (layer "B.Cu") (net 27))
 (segment (start 128.668 118.609) (end 131.478 118.609) (width 0.25) (layer "B.Cu") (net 27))
 (segment (start 126.538 114.564) (end 126.893 114.564) (width 0.25) (layer "F.Cu") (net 3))
 (segment (start 123.348 119.809) (end 123.348 121.789) (width 0.25) (layer "F.Cu") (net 3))
 (segment (start 120.948 121.789) (end 118.798 119.639) (width 0.25) (layer "F.Cu") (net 3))
 (segment (start 125.778 121.019) (end 125.798 121.019) (width 0.25) (layer "F.Cu") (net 3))
 (segment (start 126.198 120.619) (end 126.198 120.259) (width 0.25) (layer "F.Cu") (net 3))
 (segment (start 123.348 121.789) (end 125.008 121.789) (width 0.25) (layer "F.Cu") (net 3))
 (segment (start 125.798 121.019) (end 126.198 120.619) (width 0.25) (layer "F.Cu") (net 3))
 (segment (start 125.008 121.789) (end 125.778 121.019) (width 0.25) (layer "F.Cu") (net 3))
 (segment (start 123.348 121.789) (end 120.948 121.789) (width 0.25) (layer "F.Cu") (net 3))
 (segment (start 126.893 114.564) (end 126.898 114.559) (width 0.25) (layer "F.Cu") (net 3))
 (via (at 126.898 114.559) (size 0.8) (drill 0.4) (layers "F.Cu" "B.Cu") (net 3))
 (via (at 118.798 119.639) (size 0.8) (drill 0.4) (layers "F.Cu" "B.Cu") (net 3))
 (segment (start 131.268 119.459) (end 131.498 119.229) (width 0.25) (layer "B.Cu") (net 3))
 (segment (start 119.708 107.194) (end 114.993 111.909) (width 0.512) (layer "B.Cu") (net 3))
 (segment (start 125.003 107.194) (end 119.708 107.194) (width 0.512) (layer "B.Cu") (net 3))
 (segment (start 107.493 104.409) (end 107.493 105.921) (width 0.512) (layer "B.Cu") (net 3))
 (segment (start 122.548 119.459) (end 131.268 119.459) (width 0.25) (layer "B.Cu") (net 3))
 (segment (start 107.493 119.409) (end 114.993 111.909) (width 0.512) (layer "B.Cu") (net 3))
 (segment (start 127.723 113.734) (end 127.723 107.194) (width 0.25) (layer "B.Cu") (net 3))
 (segment (start 122.518 119.429) (end 122.513 119.429) (width 0.254) (layer "B.Cu") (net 3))
 (segment (start 122.518 119.429) (end 122.548 119.459) (width 0.25) (layer "B.Cu") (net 3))
 (segment (start 131.483 107.194) (end 127.723 107.194) (width 0.25) (layer "B.Cu") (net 3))
 (segment (start 126.898 114.559) (end 127.723 113.734) (width 0.25) (layer "B.Cu") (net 3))
 (segment (start 107.493 105.921) (end 113.481 111.909) (width 0.512) (layer "B.Cu") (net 3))
 (segment (start 107.493 121.409) (end 107.493 119.409) (width 0.512) (layer "B.Cu") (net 3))
 (segment (start 113.481 111.909) (end 114.993 111.909) (width 0.512) (layer "B.Cu") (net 3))
 (segment (start 131.638 107.349) (end 131.483 107.194) (width 0.25) (layer "B.Cu") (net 3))
 (segment (start 122.513 119.429) (end 114.993 111.909) (width 0.254) (layer "B.Cu") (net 3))
 (segment (start 127.723 107.194) (end 125.003 107.194) (width 0.25) (layer "B.Cu") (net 3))
 (segment (start 128.028 118.609) (end 128.013 118.624) (width 0.25) (layer "B.Cu") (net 28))
 (segment (start 128.013 118.624) (end 125.003 118.624) (width 0.25) (layer "B.Cu") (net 28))
 (segment (start 124.003 104.409) (end 124.503 103.909) (width 0.25) (layer "B.Cu") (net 32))
 (segment (start 124.503 103.909) (end 128.1105 103.909) (width 0.25) (layer "B.Cu") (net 32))
 (segment (start 124.003 121.409) (end 131.028 121.409) (width 0.25) (layer "B.Cu") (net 31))
 (segment (start 132.828 112.739) (end 131.638 111.549) (width 0.25) (layer "B.Cu") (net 31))
 (segment (start 131.028 121.409) (end 132.828 119.609) (width 0.25) (layer "B.Cu") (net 31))
 (segment (start 132.828 119.609) (end 132.828 112.739) (width 0.25) (layer "B.Cu") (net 31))
 (segment (start 123.1205 106.2915) (end 121.928 105.099) (width 0.25) (layer "F.Cu") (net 13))
 (segment (start 123.1205 106.569) (end 123.1205 106.2915) (width 0.25) (layer "F.Cu") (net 13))
 (segment (start 122.278 118.509) (end 123.148 118.509) (width 0.25) (layer "F.Cu") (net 7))
 (segment (start 123.148 118.509) (end 123.348 118.309) (width 0.25) (layer "F.Cu") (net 7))
 (segment (start 122.258 117.484) (end 121.638 118.104) (width 0.25) (layer "F.Cu") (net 16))
 (segment (start 121.638 118.104) (end 121.638 118.509) (width 0.25) (layer "F.Cu") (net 16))
 (segment (start 118.918 111.254) (end 118.918 109.3465) (width 0.25) (layer "F.Cu") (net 26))
 (segment (start 120.675 109.108) (end 121.6955 108.0875) (width 0.25) (layer "F.Cu") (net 26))
 (segment (start 118.918 109.3465) (end 119.1565 109.108) (width 0.25) (layer "F.Cu") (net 26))
 (segment (start 119.1565 109.108) (end 120.675 109.108) (width 0.25) (layer "F.Cu") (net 26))
 (segment (start 121.6955 108.0875) (end 121.6955 106.569) (width 0.25) (layer "F.Cu") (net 26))
 (segment (start 123.998 111.254) (end 123.998 115.104) (width 0.25) (layer "F.Cu") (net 17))
 (segment (start 123.998 115.104) (end 122.258 116.844) (width 0.25) (layer "F.Cu") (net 17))
 (segment (start 121.213 116.796) (end 121.213 114.809) (width 0.25) (layer "F.Cu") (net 20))
 (segment (start 121.213 114.809) (end 121.458 114.564) (width 0.25) (layer "F.Cu") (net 20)))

